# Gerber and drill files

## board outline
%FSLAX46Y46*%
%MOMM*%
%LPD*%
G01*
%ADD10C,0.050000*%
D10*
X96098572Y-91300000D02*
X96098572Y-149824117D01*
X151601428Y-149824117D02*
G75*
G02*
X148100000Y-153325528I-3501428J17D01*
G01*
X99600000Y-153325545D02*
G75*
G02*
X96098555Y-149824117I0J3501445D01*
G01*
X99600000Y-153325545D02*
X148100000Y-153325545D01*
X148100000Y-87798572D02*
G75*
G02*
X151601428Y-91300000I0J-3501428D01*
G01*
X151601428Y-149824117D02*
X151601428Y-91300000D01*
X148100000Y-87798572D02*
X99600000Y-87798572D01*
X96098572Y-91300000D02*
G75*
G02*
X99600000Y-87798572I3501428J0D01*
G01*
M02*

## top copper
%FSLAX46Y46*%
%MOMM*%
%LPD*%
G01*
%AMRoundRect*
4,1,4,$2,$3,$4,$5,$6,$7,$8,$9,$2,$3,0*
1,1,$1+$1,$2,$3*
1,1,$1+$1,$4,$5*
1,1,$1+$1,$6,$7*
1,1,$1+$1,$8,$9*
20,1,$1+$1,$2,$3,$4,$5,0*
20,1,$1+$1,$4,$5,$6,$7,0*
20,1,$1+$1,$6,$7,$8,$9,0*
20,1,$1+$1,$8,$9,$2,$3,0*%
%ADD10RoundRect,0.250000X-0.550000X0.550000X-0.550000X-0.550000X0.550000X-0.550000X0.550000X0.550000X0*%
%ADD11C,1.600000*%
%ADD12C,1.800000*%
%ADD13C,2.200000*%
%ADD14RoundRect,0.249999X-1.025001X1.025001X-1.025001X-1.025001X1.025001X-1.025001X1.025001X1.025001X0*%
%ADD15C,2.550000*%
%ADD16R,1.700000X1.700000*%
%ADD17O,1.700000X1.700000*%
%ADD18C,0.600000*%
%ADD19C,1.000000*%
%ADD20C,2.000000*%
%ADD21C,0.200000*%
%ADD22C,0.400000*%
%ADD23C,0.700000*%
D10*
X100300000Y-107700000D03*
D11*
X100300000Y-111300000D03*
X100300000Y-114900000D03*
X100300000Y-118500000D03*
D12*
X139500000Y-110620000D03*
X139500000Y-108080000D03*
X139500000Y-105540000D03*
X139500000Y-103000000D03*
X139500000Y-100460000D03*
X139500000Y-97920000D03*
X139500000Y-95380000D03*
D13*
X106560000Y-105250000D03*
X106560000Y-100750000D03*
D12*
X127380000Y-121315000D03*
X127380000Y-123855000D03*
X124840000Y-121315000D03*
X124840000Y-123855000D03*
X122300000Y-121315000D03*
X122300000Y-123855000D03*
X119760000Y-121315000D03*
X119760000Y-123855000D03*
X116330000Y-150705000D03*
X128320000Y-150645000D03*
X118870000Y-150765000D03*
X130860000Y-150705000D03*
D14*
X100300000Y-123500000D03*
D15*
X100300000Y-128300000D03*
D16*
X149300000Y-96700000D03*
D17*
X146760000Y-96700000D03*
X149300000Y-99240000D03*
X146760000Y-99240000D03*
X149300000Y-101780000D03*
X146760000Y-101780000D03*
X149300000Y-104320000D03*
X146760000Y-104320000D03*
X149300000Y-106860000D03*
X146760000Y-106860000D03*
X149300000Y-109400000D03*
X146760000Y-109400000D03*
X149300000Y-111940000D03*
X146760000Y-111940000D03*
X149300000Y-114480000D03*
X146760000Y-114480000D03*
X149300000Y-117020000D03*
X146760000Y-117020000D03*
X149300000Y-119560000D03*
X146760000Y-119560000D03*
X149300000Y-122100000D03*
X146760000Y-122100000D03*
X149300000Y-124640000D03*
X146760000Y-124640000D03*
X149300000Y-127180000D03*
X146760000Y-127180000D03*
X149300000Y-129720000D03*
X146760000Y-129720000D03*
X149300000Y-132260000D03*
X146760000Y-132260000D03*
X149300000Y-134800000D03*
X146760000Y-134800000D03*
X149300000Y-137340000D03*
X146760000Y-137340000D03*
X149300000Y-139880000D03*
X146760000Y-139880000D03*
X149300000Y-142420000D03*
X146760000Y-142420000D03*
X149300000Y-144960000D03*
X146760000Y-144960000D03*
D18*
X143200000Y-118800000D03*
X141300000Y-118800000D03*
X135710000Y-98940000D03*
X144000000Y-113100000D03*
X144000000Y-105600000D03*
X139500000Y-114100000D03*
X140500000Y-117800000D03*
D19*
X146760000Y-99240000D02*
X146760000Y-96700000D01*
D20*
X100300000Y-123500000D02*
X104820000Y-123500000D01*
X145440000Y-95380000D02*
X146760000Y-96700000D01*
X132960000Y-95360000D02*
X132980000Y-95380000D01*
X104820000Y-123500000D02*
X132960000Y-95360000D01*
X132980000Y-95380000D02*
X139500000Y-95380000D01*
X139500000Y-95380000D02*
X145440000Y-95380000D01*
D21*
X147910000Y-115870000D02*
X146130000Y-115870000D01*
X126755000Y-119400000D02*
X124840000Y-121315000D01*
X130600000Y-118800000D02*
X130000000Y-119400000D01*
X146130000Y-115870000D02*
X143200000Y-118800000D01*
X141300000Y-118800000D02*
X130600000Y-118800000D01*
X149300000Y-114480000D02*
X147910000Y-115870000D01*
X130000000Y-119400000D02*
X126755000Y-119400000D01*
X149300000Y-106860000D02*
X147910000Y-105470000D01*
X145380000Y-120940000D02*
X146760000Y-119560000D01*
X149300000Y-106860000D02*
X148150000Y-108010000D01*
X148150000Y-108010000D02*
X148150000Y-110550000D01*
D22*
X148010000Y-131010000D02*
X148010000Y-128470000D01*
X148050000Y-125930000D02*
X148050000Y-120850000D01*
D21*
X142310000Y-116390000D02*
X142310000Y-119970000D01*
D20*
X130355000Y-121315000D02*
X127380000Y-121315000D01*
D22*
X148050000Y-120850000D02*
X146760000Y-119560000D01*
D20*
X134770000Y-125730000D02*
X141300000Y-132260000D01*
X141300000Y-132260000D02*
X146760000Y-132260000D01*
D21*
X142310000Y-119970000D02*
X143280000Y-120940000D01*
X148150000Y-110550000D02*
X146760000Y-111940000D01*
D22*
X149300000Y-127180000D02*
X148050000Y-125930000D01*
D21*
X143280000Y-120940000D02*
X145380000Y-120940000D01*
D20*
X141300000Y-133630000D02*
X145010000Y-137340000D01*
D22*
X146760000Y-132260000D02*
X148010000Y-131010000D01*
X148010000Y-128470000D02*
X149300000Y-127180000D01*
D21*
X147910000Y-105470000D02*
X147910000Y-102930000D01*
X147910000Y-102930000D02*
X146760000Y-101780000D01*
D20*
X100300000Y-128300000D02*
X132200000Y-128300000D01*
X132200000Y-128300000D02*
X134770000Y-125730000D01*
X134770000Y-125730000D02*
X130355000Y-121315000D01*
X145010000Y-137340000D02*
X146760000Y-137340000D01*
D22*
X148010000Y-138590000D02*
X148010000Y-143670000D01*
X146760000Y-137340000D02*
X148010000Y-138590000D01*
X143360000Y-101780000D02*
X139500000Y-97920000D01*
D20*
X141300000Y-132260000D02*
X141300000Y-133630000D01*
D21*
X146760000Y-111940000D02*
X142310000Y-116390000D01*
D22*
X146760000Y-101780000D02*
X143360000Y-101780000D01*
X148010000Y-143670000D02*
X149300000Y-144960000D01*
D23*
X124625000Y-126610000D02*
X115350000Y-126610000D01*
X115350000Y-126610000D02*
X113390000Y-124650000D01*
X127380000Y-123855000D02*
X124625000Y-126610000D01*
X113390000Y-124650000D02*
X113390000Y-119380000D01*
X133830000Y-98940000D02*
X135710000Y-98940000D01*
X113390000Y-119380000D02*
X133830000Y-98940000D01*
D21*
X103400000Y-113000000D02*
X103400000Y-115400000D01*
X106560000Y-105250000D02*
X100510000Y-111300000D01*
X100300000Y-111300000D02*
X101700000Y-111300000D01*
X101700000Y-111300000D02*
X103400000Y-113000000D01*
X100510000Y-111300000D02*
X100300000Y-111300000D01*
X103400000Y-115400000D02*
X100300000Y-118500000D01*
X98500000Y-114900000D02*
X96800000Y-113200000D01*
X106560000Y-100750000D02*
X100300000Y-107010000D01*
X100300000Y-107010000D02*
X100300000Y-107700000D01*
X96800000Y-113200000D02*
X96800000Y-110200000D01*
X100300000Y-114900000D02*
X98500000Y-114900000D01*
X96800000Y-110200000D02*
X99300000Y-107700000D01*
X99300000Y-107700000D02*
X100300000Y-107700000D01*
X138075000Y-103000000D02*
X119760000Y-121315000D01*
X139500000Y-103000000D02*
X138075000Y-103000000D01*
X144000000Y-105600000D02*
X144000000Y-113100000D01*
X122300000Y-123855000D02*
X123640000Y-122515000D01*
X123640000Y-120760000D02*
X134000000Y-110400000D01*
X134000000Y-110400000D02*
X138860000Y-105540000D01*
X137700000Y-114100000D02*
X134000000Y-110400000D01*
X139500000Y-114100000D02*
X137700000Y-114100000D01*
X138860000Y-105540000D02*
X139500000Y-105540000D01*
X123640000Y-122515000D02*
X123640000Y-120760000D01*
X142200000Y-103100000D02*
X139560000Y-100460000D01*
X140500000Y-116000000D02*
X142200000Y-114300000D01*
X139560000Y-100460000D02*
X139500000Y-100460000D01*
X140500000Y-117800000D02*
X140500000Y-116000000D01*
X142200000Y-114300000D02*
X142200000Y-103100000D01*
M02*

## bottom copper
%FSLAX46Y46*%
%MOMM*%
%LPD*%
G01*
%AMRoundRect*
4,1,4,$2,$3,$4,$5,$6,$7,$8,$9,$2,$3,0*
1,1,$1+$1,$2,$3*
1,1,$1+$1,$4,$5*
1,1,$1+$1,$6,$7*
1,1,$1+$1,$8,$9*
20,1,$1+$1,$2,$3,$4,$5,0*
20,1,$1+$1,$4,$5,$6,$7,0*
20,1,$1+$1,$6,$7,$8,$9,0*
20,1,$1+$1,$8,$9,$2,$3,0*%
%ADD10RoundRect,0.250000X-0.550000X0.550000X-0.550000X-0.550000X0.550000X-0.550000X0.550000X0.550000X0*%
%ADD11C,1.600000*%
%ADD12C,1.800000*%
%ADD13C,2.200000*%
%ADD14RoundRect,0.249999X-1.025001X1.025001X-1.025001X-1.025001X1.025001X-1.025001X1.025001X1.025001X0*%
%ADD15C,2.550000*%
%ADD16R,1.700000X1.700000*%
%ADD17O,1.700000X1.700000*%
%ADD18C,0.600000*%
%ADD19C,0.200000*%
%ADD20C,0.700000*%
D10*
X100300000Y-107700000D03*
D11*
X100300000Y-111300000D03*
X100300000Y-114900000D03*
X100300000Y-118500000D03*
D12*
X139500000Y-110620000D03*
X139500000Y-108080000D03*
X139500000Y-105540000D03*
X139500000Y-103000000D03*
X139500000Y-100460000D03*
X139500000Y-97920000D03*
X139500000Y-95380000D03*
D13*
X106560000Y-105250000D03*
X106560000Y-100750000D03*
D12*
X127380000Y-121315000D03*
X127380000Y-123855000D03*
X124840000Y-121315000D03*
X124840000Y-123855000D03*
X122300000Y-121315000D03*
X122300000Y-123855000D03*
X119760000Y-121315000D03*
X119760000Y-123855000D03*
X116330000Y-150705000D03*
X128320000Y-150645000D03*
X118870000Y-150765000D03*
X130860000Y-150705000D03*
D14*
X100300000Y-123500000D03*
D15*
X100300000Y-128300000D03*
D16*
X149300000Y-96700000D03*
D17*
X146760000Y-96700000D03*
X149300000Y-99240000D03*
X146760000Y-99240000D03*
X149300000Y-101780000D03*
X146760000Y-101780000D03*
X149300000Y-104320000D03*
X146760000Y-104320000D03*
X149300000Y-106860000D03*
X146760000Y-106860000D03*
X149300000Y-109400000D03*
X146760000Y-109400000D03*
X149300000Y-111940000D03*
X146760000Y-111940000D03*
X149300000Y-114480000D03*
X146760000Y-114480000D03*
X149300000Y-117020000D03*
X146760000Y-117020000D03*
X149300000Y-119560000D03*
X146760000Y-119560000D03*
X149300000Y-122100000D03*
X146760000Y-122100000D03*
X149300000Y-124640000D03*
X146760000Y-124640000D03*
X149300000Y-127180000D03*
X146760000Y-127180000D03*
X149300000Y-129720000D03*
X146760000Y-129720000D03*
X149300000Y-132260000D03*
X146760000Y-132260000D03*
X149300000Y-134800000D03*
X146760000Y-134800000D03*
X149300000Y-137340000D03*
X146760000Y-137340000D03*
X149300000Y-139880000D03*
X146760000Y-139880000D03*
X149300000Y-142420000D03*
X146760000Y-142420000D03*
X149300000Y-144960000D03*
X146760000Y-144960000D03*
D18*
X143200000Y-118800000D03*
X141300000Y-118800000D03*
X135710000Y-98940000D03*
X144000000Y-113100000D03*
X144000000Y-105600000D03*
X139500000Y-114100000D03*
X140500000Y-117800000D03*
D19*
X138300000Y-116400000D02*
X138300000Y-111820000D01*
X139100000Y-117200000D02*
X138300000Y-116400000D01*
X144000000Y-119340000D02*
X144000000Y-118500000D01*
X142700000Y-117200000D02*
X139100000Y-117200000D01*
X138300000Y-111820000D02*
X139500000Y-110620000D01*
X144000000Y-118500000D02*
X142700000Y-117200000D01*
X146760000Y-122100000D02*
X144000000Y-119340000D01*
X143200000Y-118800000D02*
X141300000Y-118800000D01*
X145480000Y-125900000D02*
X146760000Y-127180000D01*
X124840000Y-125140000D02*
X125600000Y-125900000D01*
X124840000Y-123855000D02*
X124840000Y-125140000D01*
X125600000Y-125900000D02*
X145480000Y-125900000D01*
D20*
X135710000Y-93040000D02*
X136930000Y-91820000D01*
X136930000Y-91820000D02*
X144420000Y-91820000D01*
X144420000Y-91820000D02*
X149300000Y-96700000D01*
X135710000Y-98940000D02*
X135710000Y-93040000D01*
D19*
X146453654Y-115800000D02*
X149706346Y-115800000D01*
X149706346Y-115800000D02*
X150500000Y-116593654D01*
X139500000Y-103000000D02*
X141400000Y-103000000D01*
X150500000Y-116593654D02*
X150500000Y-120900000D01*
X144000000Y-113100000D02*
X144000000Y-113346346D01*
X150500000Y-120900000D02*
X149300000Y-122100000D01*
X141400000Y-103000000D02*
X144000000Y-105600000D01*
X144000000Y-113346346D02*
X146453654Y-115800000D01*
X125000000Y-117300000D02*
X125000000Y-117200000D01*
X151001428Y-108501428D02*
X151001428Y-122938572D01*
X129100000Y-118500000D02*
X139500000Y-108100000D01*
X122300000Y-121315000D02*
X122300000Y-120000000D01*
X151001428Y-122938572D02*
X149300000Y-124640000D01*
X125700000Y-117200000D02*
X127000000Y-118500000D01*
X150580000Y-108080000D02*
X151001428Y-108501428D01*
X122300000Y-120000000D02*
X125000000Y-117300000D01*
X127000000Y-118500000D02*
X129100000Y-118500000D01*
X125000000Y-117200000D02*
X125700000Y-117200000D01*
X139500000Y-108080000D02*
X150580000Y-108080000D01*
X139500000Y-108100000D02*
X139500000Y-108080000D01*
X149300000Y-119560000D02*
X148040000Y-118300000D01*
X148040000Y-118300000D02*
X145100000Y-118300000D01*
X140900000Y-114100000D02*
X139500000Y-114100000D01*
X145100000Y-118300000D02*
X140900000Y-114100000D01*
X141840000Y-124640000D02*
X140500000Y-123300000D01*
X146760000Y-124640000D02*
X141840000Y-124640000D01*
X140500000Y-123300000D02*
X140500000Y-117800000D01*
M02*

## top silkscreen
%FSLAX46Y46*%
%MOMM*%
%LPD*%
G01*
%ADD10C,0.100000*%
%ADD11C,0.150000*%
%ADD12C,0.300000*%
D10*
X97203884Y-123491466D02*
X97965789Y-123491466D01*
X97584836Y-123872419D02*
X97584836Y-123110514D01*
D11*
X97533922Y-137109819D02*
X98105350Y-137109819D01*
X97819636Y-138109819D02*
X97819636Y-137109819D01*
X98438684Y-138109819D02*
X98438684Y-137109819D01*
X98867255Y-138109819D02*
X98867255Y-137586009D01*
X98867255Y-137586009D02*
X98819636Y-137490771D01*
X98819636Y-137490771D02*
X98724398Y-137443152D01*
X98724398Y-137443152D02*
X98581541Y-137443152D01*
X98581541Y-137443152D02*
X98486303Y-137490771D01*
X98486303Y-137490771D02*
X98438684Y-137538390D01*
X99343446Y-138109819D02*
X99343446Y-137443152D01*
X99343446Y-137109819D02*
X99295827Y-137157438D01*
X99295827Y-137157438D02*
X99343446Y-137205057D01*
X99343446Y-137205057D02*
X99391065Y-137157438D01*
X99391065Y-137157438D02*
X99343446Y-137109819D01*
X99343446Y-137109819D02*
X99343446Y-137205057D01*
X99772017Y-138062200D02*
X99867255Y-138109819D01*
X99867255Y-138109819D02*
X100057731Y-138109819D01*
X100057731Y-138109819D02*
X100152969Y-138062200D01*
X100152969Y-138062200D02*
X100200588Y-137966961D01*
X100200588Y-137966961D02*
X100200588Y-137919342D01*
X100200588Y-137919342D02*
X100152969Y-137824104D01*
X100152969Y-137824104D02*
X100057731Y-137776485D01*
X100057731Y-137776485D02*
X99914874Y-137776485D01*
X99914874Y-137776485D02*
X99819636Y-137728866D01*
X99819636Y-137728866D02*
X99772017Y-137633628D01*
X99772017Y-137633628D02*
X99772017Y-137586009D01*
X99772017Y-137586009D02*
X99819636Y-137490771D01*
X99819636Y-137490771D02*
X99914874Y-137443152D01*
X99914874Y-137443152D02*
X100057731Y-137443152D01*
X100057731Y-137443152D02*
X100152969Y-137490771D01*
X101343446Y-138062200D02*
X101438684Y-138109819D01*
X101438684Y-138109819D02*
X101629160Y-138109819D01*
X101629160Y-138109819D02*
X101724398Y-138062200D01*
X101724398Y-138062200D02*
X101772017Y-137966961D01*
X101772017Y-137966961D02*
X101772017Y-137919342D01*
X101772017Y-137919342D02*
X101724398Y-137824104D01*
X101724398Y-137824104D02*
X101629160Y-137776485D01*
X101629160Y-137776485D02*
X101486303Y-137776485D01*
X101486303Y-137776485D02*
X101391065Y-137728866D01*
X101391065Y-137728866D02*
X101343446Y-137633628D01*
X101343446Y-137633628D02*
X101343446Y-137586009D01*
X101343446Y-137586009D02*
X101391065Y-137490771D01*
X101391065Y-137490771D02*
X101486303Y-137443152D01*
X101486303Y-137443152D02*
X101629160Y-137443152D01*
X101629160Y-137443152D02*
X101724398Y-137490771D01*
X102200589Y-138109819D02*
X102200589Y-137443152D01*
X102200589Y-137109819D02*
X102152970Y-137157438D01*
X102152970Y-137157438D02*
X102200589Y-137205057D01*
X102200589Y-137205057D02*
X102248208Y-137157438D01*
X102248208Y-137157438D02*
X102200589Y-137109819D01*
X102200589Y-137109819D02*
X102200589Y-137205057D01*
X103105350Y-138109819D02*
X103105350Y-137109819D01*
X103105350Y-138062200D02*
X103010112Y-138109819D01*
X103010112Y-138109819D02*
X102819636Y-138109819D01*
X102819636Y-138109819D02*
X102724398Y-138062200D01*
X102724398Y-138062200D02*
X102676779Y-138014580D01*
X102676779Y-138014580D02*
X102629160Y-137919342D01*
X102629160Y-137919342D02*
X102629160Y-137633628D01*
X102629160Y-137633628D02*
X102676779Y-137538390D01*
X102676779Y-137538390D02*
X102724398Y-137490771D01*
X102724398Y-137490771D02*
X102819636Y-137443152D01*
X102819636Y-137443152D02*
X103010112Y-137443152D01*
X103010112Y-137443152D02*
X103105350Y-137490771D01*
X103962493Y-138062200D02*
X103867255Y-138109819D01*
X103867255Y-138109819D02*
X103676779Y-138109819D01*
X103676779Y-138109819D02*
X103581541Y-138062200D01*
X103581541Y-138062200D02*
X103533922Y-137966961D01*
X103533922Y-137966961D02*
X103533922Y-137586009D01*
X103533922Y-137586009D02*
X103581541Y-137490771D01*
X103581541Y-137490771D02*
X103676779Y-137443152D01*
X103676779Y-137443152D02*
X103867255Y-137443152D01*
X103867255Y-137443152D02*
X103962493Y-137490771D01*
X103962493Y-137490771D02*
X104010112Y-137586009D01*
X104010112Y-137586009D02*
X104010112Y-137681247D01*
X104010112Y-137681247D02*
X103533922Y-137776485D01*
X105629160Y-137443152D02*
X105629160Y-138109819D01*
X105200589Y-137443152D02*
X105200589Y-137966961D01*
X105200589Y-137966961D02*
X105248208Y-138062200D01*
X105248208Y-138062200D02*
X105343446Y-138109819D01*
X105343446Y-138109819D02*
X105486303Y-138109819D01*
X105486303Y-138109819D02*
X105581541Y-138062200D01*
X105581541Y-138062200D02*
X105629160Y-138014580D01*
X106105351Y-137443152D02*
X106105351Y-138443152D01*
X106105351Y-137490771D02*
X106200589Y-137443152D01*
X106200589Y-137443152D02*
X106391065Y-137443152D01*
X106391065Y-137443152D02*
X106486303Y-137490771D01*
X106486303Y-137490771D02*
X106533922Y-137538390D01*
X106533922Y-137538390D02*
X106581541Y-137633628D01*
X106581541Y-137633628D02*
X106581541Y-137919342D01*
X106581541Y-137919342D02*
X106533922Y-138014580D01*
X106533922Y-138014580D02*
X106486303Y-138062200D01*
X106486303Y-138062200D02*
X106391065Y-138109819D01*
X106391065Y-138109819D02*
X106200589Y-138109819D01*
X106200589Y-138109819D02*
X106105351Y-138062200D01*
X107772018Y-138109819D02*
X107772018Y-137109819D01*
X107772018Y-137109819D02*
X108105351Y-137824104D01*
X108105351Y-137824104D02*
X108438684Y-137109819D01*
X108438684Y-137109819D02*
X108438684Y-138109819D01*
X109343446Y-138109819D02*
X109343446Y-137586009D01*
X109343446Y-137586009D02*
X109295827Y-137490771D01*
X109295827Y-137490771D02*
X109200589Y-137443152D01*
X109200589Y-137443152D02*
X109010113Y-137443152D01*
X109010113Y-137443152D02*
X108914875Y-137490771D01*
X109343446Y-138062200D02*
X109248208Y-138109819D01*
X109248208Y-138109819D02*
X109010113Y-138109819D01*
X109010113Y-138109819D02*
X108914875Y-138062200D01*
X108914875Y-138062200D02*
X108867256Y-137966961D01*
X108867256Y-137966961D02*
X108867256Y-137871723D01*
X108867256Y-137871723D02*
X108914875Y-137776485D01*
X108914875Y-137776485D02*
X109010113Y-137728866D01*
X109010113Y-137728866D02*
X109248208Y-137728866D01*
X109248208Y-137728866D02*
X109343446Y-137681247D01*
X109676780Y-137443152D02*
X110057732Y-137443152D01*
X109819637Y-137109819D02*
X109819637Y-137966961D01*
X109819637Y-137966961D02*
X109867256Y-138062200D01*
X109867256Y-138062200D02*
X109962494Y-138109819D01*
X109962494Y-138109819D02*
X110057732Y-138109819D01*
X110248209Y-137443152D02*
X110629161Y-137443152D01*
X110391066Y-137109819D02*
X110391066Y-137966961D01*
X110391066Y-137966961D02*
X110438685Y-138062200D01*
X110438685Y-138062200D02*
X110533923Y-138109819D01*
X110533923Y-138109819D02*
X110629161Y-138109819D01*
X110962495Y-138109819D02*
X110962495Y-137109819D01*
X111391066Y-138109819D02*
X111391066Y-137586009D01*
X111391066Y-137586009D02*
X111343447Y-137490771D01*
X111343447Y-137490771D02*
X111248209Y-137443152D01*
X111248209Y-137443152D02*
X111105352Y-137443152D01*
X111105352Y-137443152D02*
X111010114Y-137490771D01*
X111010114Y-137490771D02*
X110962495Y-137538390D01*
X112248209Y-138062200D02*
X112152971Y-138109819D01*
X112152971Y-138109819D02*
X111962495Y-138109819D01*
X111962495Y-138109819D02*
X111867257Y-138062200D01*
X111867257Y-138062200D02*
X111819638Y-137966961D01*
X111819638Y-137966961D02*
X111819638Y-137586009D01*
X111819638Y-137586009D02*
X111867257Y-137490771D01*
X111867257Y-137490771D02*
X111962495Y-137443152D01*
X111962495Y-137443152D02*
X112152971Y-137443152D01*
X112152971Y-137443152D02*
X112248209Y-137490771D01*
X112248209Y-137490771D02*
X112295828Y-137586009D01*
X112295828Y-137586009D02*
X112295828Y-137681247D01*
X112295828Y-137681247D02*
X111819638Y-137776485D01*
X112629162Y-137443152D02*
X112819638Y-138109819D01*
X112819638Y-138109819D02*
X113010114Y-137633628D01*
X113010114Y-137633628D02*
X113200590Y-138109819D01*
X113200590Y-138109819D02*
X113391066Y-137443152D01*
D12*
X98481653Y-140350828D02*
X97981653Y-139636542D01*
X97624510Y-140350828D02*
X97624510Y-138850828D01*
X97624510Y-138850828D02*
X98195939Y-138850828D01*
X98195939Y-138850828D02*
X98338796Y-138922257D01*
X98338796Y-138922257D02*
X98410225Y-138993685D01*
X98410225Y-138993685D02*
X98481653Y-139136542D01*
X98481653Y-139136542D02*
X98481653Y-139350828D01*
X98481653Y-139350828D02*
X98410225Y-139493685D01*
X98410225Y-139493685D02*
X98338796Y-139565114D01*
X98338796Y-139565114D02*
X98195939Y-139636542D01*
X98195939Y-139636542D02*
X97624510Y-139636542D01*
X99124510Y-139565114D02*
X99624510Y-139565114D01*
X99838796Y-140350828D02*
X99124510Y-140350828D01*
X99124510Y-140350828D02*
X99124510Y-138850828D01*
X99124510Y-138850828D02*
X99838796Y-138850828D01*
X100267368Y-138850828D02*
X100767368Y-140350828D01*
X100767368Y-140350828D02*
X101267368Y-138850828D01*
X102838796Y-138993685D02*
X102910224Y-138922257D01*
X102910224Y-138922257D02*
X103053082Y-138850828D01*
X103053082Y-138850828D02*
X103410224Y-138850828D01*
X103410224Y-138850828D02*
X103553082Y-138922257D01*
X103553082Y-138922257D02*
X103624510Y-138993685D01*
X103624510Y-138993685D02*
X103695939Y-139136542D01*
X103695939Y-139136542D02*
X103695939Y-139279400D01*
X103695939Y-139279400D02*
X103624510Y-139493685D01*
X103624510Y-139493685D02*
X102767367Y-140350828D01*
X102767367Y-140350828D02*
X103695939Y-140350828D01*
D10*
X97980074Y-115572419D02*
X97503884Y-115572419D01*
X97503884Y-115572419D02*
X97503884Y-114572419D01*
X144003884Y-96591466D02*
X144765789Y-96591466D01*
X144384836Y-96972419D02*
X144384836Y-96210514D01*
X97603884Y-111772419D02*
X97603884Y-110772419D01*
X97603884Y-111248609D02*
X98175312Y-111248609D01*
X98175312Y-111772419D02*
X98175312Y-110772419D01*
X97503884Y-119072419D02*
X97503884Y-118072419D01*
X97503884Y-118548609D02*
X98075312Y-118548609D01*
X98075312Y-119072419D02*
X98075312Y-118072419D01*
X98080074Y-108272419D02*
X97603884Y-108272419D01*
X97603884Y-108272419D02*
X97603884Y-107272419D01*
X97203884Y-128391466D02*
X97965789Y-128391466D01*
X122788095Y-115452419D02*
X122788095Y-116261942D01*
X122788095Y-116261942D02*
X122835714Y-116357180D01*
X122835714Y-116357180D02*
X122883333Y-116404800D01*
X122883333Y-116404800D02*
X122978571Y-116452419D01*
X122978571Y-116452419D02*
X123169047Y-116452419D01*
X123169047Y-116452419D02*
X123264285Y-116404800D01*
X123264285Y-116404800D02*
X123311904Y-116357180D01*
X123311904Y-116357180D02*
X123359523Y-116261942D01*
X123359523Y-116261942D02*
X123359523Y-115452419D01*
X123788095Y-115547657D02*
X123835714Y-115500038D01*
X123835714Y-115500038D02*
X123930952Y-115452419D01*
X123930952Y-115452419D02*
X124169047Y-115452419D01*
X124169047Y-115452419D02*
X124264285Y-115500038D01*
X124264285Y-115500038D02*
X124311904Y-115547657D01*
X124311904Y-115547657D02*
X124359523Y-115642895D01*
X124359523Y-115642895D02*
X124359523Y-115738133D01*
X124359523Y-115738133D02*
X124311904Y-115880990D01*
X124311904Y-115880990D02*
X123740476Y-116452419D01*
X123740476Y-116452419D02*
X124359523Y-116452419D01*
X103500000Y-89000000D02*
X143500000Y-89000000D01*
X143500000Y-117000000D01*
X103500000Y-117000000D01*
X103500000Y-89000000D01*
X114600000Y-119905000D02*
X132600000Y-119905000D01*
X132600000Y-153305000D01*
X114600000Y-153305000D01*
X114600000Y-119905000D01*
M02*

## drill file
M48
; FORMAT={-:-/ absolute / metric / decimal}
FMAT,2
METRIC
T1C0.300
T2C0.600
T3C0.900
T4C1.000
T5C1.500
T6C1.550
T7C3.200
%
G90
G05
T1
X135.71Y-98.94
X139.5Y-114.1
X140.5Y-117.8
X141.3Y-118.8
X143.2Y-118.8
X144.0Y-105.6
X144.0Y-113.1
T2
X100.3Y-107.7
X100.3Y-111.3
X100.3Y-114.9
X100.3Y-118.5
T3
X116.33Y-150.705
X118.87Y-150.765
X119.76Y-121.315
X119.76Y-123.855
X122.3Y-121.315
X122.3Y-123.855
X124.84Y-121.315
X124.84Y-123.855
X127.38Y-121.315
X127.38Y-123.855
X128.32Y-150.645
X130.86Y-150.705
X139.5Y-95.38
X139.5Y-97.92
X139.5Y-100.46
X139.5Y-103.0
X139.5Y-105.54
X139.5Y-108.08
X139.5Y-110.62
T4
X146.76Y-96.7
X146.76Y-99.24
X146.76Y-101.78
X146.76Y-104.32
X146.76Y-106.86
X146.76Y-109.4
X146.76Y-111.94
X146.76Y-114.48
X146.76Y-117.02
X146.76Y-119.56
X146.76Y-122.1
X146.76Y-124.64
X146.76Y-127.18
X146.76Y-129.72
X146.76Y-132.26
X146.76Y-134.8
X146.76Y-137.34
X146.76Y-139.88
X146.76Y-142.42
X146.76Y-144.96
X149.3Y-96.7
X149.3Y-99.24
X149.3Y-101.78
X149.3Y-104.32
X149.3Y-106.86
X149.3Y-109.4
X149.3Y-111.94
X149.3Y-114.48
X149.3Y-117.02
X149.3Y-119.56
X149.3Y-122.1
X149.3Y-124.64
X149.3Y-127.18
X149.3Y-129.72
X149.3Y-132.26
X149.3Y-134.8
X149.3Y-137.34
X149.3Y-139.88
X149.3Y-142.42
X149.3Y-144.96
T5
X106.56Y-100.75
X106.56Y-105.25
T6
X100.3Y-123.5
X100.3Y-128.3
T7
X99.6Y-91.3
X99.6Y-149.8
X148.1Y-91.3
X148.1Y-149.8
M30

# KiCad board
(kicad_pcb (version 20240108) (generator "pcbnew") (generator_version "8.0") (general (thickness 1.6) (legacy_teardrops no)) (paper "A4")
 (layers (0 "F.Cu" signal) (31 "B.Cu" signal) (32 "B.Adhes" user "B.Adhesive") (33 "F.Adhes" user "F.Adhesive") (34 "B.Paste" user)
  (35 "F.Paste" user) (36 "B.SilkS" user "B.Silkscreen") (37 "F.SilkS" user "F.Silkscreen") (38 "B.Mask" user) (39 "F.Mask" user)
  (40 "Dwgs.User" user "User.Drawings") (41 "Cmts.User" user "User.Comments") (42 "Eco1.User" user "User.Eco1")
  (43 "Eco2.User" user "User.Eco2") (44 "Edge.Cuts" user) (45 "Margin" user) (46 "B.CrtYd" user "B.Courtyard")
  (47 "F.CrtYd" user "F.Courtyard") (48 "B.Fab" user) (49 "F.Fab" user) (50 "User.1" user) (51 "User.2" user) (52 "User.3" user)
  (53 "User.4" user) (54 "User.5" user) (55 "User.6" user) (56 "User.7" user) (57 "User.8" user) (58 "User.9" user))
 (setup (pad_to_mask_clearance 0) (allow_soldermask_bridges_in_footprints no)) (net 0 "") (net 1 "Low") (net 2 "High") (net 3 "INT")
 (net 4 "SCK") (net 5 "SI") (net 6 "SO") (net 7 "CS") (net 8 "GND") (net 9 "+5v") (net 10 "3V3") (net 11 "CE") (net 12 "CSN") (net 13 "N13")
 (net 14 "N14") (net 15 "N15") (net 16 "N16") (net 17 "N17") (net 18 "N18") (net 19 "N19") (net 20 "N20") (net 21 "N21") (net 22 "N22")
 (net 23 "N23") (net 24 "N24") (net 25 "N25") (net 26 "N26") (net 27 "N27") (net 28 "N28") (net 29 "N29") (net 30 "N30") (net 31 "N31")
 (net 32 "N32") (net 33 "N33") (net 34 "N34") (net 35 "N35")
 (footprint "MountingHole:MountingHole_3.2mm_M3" (layer "F.Cu") (at 148.1 91.3 180)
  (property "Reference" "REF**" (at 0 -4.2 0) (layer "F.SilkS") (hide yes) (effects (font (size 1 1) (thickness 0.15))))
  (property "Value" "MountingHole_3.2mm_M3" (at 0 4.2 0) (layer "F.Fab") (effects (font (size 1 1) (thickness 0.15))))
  (pad "" np_thru_hole circle (at 0 0 180) (size 3.2 3.2) (drill 3.2) (layers "*.Cu" "*.Mask")))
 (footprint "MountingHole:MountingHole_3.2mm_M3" (layer "F.Cu") (at 99.6 91.3 180)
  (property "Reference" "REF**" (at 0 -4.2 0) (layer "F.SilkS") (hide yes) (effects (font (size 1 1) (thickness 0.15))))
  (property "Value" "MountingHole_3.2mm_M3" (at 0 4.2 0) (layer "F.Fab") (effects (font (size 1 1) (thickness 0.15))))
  (pad "" np_thru_hole circle (at 0 0 180) (size 3.2 3.2) (drill 3.2) (layers "*.Cu" "*.Mask")))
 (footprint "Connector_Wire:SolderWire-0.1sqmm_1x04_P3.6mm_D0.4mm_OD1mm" (layer "F.Cu") (at 100.3 107.7 -90)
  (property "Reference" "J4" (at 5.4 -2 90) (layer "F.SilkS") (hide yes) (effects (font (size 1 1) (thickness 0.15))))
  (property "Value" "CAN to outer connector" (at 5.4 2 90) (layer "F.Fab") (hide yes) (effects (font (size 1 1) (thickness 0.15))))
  (pad "1" thru_hole roundrect (at 0 0 270) (size 1.6 1.6) (drill 0.6) (layers "*.Cu" "*.Mask") (remove_unused_layers no)
   (roundrect_rratio 0.15625) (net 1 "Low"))
  (pad "2" thru_hole circle (at 3.6 0 270) (size 1.6 1.6) (drill 0.6) (layers "*.Cu" "*.Mask") (remove_unused_layers no) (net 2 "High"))
  (pad "3" thru_hole circle (at 7.2 0 270) (size 1.6 1.6) (drill 0.6) (layers "*.Cu" "*.Mask") (remove_unused_layers no) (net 1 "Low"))
  (pad "4" thru_hole circle (at 10.8 0 270) (size 1.6 1.6) (drill 0.6) (layers "*.Cu" "*.Mask") (remove_unused_layers no) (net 2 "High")))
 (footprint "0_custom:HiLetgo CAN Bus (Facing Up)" (layer "F.Cu") (at 129.55 100.6 180)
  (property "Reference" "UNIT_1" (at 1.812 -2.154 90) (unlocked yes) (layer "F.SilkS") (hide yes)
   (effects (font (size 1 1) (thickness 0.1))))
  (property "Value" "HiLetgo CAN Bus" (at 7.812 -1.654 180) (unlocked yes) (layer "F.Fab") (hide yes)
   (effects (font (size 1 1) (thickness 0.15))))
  (fp_rect (start -13.95 -16.4) (end 26.05 11.6) (stroke (width 0.1) (type default)) (fill none) (layer "F.SilkS"))
  (pad "1" thru_hole circle (at -9.95 -10.02) (size 1.8 1.8) (drill 0.9) (layers "*.Cu" "*.Mask") (remove_unused_layers no) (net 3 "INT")
   (solder_mask_margin 0.102))
  (pad "2" thru_hole circle (at -9.95 -7.48) (size 1.8 1.8) (drill 0.9) (layers "*.Cu" "*.Mask") (remove_unused_layers no) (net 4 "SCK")
   (solder_mask_margin 0.102))
  (pad "3" thru_hole circle (at -9.95 -4.94) (size 1.8 1.8) (drill 0.9) (layers "*.Cu" "*.Mask") (remove_unused_layers no) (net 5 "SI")
   (solder_mask_margin 0.102))
  (pad "4" thru_hole circle (at -9.95 -2.4) (size 1.8 1.8) (drill 0.9) (layers "*.Cu" "*.Mask") (remove_unused_layers no) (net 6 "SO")
   (solder_mask_margin 0.102))
  (pad "5" thru_hole circle (at -9.95 0.14) (size 1.8 1.8) (drill 0.9) (layers "*.Cu" "*.Mask") (remove_unused_layers no) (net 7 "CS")
   (solder_mask_margin 0.102))
  (pad "6" thru_hole circle (at -9.95 2.68) (size 1.8 1.8) (drill 0.9) (layers "*.Cu" "*.Mask") (remove_unused_layers no) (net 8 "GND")
   (solder_mask_margin 0.102))
  (pad "7" thru_hole circle (at -9.95 5.22) (size 1.8 1.8) (drill 0.9) (layers "*.Cu" "*.Mask") (remove_unused_layers no) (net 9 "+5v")
   (solder_mask_margin 0.102))
  (pad "8" thru_hole circle (at 22.99 -4.65) (size 2.2 2.2) (drill 1.5) (layers "*.Cu" "*.Mask") (remove_unused_layers no) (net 2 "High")
   (solder_mask_margin 0.102))
  (pad "9" thru_hole circle (at 22.99 -0.15) (size 2.2 2.2) (drill 1.5) (layers "*.Cu" "*.Mask") (remove_unused_layers no) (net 1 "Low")
   (solder_mask_margin 0.102)))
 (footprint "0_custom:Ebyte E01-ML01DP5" (layer "F.Cu") (at 123.55 116.495)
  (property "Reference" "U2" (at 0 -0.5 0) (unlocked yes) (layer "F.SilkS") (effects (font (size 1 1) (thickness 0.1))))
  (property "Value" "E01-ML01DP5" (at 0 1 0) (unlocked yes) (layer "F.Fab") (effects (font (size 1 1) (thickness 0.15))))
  (fp_rect (start -8.95 3.41) (end 9.05 36.81) (stroke (width 0.1) (type default)) (fill none) (layer "F.SilkS"))
  (pad "1" thru_hole circle (at 3.83 4.82 180) (size 1.8 1.8) (drill 0.9) (layers "*.Cu" "*.Mask") (remove_unused_layers no) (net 8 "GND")
   (solder_mask_margin 0.102))
  (pad "2" thru_hole circle (at 3.83 7.36 180) (size 1.8 1.8) (drill 0.9) (layers "*.Cu" "*.Mask") (remove_unused_layers no) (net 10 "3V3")
   (solder_mask_margin 0.102))
  (pad "3" thru_hole circle (at 1.29 4.82 180) (size 1.8 1.8) (drill 0.9) (layers "*.Cu" "*.Mask") (remove_unused_layers no) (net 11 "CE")
   (solder_mask_margin 0.102))
  (pad "4" thru_hole circle (at 1.29 7.36 180) (size 1.8 1.8) (drill 0.9) (layers "*.Cu" "*.Mask") (remove_unused_layers no) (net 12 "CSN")
   (solder_mask_margin 0.102))
  (pad "5" thru_hole circle (at -1.25 4.82 180) (size 1.8 1.8) (drill 0.9) (layers "*.Cu" "*.Mask") (remove_unused_layers no) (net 4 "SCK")
   (solder_mask_margin 0.102))
  (pad "6" thru_hole circle (at -1.25 7.36 180) (size 1.8 1.8) (drill 0.9) (layers "*.Cu" "*.Mask") (remove_unused_layers no) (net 5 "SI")
   (solder_mask_margin 0.102))
  (pad "7" thru_hole circle (at -3.79 4.82 90) (size 1.8 1.8) (drill 0.9) (layers "*.Cu" "*.Mask") (remove_unused_layers no) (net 6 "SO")
   (solder_mask_margin 0.102))
  (pad "8" thru_hole circle (at -3.79 7.36 90) (size 1.8 1.8) (drill 0.9) (layers "*.Cu" "*.Mask") (remove_unused_layers no) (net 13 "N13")
   (solder_mask_margin 0.102))
  (pad "9" thru_hole circle (at -7.22 34.21 270) (size 1.8 1.8) (drill 0.9) (layers "*.Cu" "*.Mask") (remove_unused_layers no)
   (solder_mask_margin 0.102))
  (pad "9" thru_hole circle (at 4.77 34.15 270) (size 1.8 1.8) (drill 0.9) (layers "*.Cu" "*.Mask") (remove_unused_layers no)
   (solder_mask_margin 0.102))
  (pad "10" thru_hole circle (at -4.68 34.27 270) (size 1.8 1.8) (drill 0.9) (layers "*.Cu" "*.Mask") (remove_unused_layers no)
   (solder_mask_margin 0.102))
  (pad "10" thru_hole circle (at 7.31 34.21 270) (size 1.8 1.8) (drill 0.9) (layers "*.Cu" "*.Mask") (remove_unused_layers no)
   (solder_mask_margin 0.102)))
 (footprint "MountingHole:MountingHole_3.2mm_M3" (layer "F.Cu") (at 99.6 149.8)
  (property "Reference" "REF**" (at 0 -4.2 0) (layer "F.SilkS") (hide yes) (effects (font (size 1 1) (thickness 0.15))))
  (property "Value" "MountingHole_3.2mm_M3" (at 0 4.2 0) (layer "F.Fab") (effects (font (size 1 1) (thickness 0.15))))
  (pad "" np_thru_hole circle (at 0 0) (size 3.2 3.2) (drill 3.2) (layers "*.Cu" "*.Mask")))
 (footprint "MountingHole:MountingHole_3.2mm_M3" (layer "F.Cu") (at 148.1 149.8)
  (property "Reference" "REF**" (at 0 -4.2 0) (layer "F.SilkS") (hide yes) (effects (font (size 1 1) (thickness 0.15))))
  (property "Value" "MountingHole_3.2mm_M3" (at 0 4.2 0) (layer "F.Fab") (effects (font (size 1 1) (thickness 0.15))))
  (pad "" np_thru_hole circle (at 0 0) (size 3.2 3.2) (drill 3.2) (layers "*.Cu" "*.Mask")))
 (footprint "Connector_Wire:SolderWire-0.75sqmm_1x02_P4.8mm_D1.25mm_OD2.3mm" (layer "F.Cu") (at 100.3 123.5 -90)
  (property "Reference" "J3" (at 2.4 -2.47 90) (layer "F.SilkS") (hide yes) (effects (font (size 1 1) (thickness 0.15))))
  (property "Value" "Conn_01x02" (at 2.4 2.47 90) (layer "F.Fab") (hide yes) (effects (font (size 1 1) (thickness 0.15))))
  (pad "1" thru_hole roundrect (at 0 0 270) (size 2.55 2.55) (drill 1.55) (layers "*.Cu" "*.Mask") (remove_unused_layers no)
   (roundrect_rratio 0.098039) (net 9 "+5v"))
  (pad "2" thru_hole circle (at 4.8 0 270) (size 2.55 2.55) (drill 1.55) (layers "*.Cu" "*.Mask") (remove_unused_layers no) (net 8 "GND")))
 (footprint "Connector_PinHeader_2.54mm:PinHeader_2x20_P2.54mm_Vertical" (layer "B.Cu") (at 149.3 96.7 180)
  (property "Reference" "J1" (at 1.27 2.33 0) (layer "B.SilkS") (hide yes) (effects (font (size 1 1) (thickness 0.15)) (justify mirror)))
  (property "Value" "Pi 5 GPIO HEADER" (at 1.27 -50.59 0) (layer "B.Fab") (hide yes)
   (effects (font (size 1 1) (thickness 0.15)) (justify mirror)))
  (pad "1" thru_hole rect (at 0 0 180) (size 1.7 1.7) (drill 1) (layers "*.Cu" "*.Mask") (remove_unused_layers no) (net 10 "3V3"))
  (pad "2" thru_hole oval (at 2.54 0 180) (size 1.7 1.7) (drill 1) (layers "*.Cu" "*.Mask") (remove_unused_layers no) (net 9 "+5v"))
  (pad "3" thru_hole oval (at 0 -2.54 180) (size 1.7 1.7) (drill 1) (layers "*.Cu" "*.Mask") (remove_unused_layers no) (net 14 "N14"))
  (pad "4" thru_hole oval (at 2.54 -2.54 180) (size 1.7 1.7) (drill 1) (layers "*.Cu" "*.Mask") (remove_unused_layers no) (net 9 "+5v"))
  (pad "5" thru_hole oval (at 0 -5.08 180) (size 1.7 1.7) (drill 1) (layers "*.Cu" "*.Mask") (remove_unused_layers no) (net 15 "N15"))
  (pad "6" thru_hole oval (at 2.54 -5.08 180) (size 1.7 1.7) (drill 1) (layers "*.Cu" "*.Mask") (remove_unused_layers no) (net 8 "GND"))
  (pad "7" thru_hole oval (at 0 -7.62 180) (size 1.7 1.7) (drill 1) (layers "*.Cu" "*.Mask") (remove_unused_layers no) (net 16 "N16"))
  (pad "8" thru_hole oval (at 2.54 -7.62 180) (size 1.7 1.7) (drill 1) (layers "*.Cu" "*.Mask") (remove_unused_layers no) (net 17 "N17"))
  (pad "9" thru_hole oval (at 0 -10.16 180) (size 1.7 1.7) (drill 1) (layers "*.Cu" "*.Mask") (remove_unused_layers no) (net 8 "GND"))
  (pad "10" thru_hole oval (at 2.54 -10.16 180) (size 1.7 1.7) (drill 1) (layers "*.Cu" "*.Mask") (remove_unused_layers no) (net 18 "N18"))
  (pad "11" thru_hole oval (at 0 -12.7 180) (size 1.7 1.7) (drill 1) (layers "*.Cu" "*.Mask") (remove_unused_layers no) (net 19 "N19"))
  (pad "12" thru_hole oval (at 2.54 -12.7 180) (size 1.7 1.7) (drill 1) (layers "*.Cu" "*.Mask") (remove_unused_layers no) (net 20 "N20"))
  (pad "13" thru_hole oval (at 0 -15.24 180) (size 1.7 1.7) (drill 1) (layers "*.Cu" "*.Mask") (remove_unused_layers no) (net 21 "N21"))
  (pad "14" thru_hole oval (at 2.54 -15.24 180) (size 1.7 1.7) (drill 1) (layers "*.Cu" "*.Mask") (remove_unused_layers no) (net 8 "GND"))
  (pad "15" thru_hole oval (at 0 -17.78 180) (size 1.7 1.7) (drill 1) (layers "*.Cu" "*.Mask") (remove_unused_layers no) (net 11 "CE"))
  (pad "16" thru_hole oval (at 2.54 -17.78 180) (size 1.7 1.7) (drill 1) (layers "*.Cu" "*.Mask") (remove_unused_layers no) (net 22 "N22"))
  (pad "17" thru_hole oval (at 0 -20.32 180) (size 1.7 1.7) (drill 1) (layers "*.Cu" "*.Mask") (remove_unused_layers no) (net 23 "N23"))
  (pad "18" thru_hole oval (at 2.54 -20.32 180) (size 1.7 1.7) (drill 1) (layers "*.Cu" "*.Mask") (remove_unused_layers no) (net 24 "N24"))
  (pad "19" thru_hole oval (at 0 -22.86 180) (size 1.7 1.7) (drill 1) (layers "*.Cu" "*.Mask") (remove_unused_layers no) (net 5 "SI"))
  (pad "20" thru_hole oval (at 2.54 -22.86 180) (size 1.7 1.7) (drill 1) (layers "*.Cu" "*.Mask") (remove_unused_layers no) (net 8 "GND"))
  (pad "21" thru_hole oval (at 0 -25.4 180) (size 1.7 1.7) (drill 1) (layers "*.Cu" "*.Mask") (remove_unused_layers no) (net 6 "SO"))
  (pad "22" thru_hole oval (at 2.54 -25.4 180) (size 1.7 1.7) (drill 1) (layers "*.Cu" "*.Mask") (remove_unused_layers no) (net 3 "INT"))
  (pad "23" thru_hole oval (at 0 -27.94 180) (size 1.7 1.7) (drill 1) (layers "*.Cu" "*.Mask") (remove_unused_layers no) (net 4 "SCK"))
  (pad "24" thru_hole oval (at 2.54 -27.94 180) (size 1.7 1.7) (drill 1) (layers "*.Cu" "*.Mask") (remove_unused_layers no) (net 7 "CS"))
  (pad "25" thru_hole oval (at 0 -30.48 180) (size 1.7 1.7) (drill 1) (layers "*.Cu" "*.Mask") (remove_unused_layers no) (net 8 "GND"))
  (pad "26" thru_hole oval (at 2.54 -30.48 180) (size 1.7 1.7) (drill 1) (layers "*.Cu" "*.Mask") (remove_unused_layers no) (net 12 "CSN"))
  (pad "27" thru_hole oval (at 0 -33.02 180) (size 1.7 1.7) (drill 1) (layers "*.Cu" "*.Mask") (remove_unused_layers no) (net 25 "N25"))
  (pad "28" thru_hole oval (at 2.54 -33.02 180) (size 1.7 1.7) (drill 1) (layers "*.Cu" "*.Mask") (remove_unused_layers no) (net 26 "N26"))
  (pad "29" thru_hole oval (at 0 -35.56 180) (size 1.7 1.7) (drill 1) (layers "*.Cu" "*.Mask") (remove_unused_layers no) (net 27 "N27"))
  (pad "30" thru_hole oval (at 2.54 -35.56 180) (size 1.7 1.7) (drill 1) (layers "*.Cu" "*.Mask") (remove_unused_layers no) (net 8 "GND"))
  (pad "31" thru_hole oval (at 0 -38.1 180) (size 1.7 1.7) (drill 1) (layers "*.Cu" "*.Mask") (remove_unused_layers no) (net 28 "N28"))
  (pad "32" thru_hole oval (at 2.54 -38.1 180) (size 1.7 1.7) (drill 1) (layers "*.Cu" "*.Mask") (remove_unused_layers no) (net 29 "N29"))
  (pad "33" thru_hole oval (at 0 -40.64 180) (size 1.7 1.7) (drill 1) (layers "*.Cu" "*.Mask") (remove_unused_layers no) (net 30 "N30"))
  (pad "34" thru_hole oval (at 2.54 -40.64 180) (size 1.7 1.7) (drill 1) (layers "*.Cu" "*.Mask") (remove_unused_layers no) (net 8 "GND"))
  (pad "35" thru_hole oval (at 0 -43.18 180) (size 1.7 1.7) (drill 1) (layers "*.Cu" "*.Mask") (remove_unused_layers no) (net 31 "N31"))
  (pad "36" thru_hole oval (at 2.54 -43.18 180) (size 1.7 1.7) (drill 1) (layers "*.Cu" "*.Mask") (remove_unused_layers no) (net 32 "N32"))
  (pad "37" thru_hole oval (at 0 -45.72 180) (size 1.7 1.7) (drill 1) (layers "*.Cu" "*.Mask") (remove_unused_layers no) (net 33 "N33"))
  (pad "38" thru_hole oval (at 2.54 -45.72 180) (size 1.7 1.7) (drill 1) (layers "*.Cu" "*.Mask") (remove_unused_layers no) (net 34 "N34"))
  (pad "39" thru_hole oval (at 0 -48.26 180) (size 1.7 1.7) (drill 1) (layers "*.Cu" "*.Mask") (remove_unused_layers no) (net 8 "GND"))
  (pad "40" thru_hole oval (at 2.54 -48.26 180) (size 1.7 1.7) (drill 1) (layers "*.Cu" "*.Mask") (remove_unused_layers no) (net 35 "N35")))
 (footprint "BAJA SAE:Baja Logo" (layer "B.Cu") (at 122.9 102.7 180)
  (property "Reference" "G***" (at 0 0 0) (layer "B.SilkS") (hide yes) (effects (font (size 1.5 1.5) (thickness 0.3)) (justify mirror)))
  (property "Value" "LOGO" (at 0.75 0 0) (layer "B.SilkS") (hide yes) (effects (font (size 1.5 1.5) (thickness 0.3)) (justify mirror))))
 (gr_line (start 96.098572 91.3) (end 96.098572 149.824117) (stroke (width 0.05) (type default)) (layer "Edge.Cuts"))
 (gr_arc (start 151.601428 149.824117) (mid 150.575883 152.3) (end 148.1 153.325545) (locked yes) (stroke (width 0.05) (type default))
  (layer "Edge.Cuts"))
 (gr_arc (start 99.6 153.325545) (mid 97.124117 152.3) (end 96.098572 149.824117) (stroke (width 0.05) (type default)) (layer "Edge.Cuts"))
 (gr_line (start 99.6 153.325545) (end 148.1 153.325545) (stroke (width 0.05) (type default)) (layer "Edge.Cuts"))
 (gr_arc (start 148.1 87.798572) (mid 150.575883 88.824117) (end 151.601428 91.3) (locked yes) (stroke (width 0.05) (type default))
  (layer "Edge.Cuts"))
 (gr_line (start 151.601428 149.824117) (end 151.601428 91.3) (stroke (width 0.05) (type default)) (layer "Edge.Cuts"))
 (gr_line (start 148.1 87.798572) (end 99.6 87.798572) (stroke (width 0.05) (type default)) (layer "Edge.Cuts"))
 (gr_arc (start 96.098572 91.3) (mid 97.124117 88.824117) (end 99.6 87.798572) (locked yes) (stroke (width 0.05) (type default))
  (layer "Edge.Cuts"))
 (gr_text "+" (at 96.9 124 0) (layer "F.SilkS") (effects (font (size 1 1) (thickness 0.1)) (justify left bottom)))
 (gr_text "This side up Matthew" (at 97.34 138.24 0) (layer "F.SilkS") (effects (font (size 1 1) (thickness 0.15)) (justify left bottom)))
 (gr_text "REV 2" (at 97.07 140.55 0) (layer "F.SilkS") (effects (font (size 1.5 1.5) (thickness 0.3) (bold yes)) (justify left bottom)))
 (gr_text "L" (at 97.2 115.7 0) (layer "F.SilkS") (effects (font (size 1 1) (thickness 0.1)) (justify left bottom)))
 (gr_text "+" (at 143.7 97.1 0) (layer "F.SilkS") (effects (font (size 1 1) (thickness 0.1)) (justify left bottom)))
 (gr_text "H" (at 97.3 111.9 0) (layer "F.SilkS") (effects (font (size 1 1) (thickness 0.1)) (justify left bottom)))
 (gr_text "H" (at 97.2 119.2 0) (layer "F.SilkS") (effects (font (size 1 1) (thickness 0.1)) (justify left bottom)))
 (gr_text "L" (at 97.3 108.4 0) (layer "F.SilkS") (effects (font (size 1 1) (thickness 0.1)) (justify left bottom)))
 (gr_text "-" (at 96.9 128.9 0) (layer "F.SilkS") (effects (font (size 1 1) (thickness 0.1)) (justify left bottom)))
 (segment (start 138.3 116.4) (end 138.3 111.82) (width 0.2) (layer "B.Cu") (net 3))
 (segment (start 139.1 117.2) (end 138.3 116.4) (width 0.2) (layer "B.Cu") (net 3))
 (segment (start 144 119.34) (end 144 118.5) (width 0.2) (layer "B.Cu") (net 3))
 (segment (start 142.7 117.2) (end 139.1 117.2) (width 0.2) (layer "B.Cu") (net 3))
 (segment (start 138.3 111.82) (end 139.5 110.62) (width 0.2) (layer "B.Cu") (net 3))
 (segment (start 144 118.5) (end 142.7 117.2) (width 0.2) (layer "B.Cu") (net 3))
 (segment (start 146.76 122.1) (end 144 119.34) (width 0.2) (layer "B.Cu") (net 3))
 (segment (start 146.76 99.24) (end 146.76 96.7) (width 1) (layer "F.Cu") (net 9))
 (segment (start 100.3 123.5) (end 104.82 123.5) (width 2) (layer "F.Cu") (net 9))
 (segment (start 145.44 95.38) (end 146.76 96.7) (width 2) (layer "F.Cu") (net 9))
 (segment (start 132.96 95.36) (end 132.98 95.38) (width 2) (layer "F.Cu") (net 9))
 (segment (start 104.82 123.5) (end 132.96 95.36) (width 2) (layer "F.Cu") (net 9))
 (segment (start 132.98 95.38) (end 139.5 95.38) (width 2) (layer "F.Cu") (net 9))
 (segment (start 139.5 95.38) (end 145.44 95.38) (width 2) (layer "F.Cu") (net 9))
 (segment (start 147.91 115.87) (end 146.13 115.87) (width 0.2) (layer "F.Cu") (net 11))
 (segment (start 126.755 119.4) (end 124.84 121.315) (width 0.2) (layer "F.Cu") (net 11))
 (segment (start 130.6 118.8) (end 130 119.4) (width 0.2) (layer "F.Cu") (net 11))
 (segment (start 146.13 115.87) (end 143.2 118.8) (width 0.2) (layer "F.Cu") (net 11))
 (segment (start 141.3 118.8) (end 130.6 118.8) (width 0.2) (layer "F.Cu") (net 11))
 (segment (start 149.3 114.48) (end 147.91 115.87) (width 0.2) (layer "F.Cu") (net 11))
 (segment (start 130 119.4) (end 126.755 119.4) (width 0.2) (layer "F.Cu") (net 11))
 (via (at 143.2 118.8) (size 0.6) (drill 0.3) (layers "F.Cu" "B.Cu") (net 11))
 (via (at 141.3 118.8) (size 0.6) (drill 0.3) (layers "F.Cu" "B.Cu") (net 11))
 (segment (start 143.2 118.8) (end 141.3 118.8) (width 0.2) (layer "B.Cu") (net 11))
 (segment (start 149.3 106.86) (end 147.91 105.47) (width 0.2) (layer "F.Cu") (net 8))
 (segment (start 145.38 120.94) (end 146.76 119.56) (width 0.2) (layer "F.Cu") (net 8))
 (segment (start 149.3 106.86) (end 148.15 108.01) (width 0.2) (layer "F.Cu") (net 8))
 (segment (start 148.15 108.01) (end 148.15 110.55) (width 0.2) (layer "F.Cu") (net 8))
 (segment (start 148.01 131.01) (end 148.01 128.47) (width 0.4) (layer "F.Cu") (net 8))
 (segment (start 148.05 125.93) (end 148.05 120.85) (width 0.4) (layer "F.Cu") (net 8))
 (segment (start 142.31 116.39) (end 142.31 119.97) (width 0.2) (layer "F.Cu") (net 8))
 (segment (start 130.355 121.315) (end 127.38 121.315) (width 2) (layer "F.Cu") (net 8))
 (segment (start 148.05 120.85) (end 146.76 119.56) (width 0.4) (layer "F.Cu") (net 8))
 (segment (start 134.77 125.73) (end 141.3 132.26) (width 2) (layer "F.Cu") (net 8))
 (segment (start 141.3 132.26) (end 146.76 132.26) (width 2) (layer "F.Cu") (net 8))
 (segment (start 142.31 119.97) (end 143.28 120.94) (width 0.2) (layer "F.Cu") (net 8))
 (segment (start 148.15 110.55) (end 146.76 111.94) (width 0.2) (layer "F.Cu") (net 8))
 (segment (start 149.3 127.18) (end 148.05 125.93) (width 0.4) (layer "F.Cu") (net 8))
 (segment (start 143.28 120.94) (end 145.38 120.94) (width 0.2) (layer "F.Cu") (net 8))
 (segment (start 141.3 133.63) (end 145.01 137.34) (width 2) (layer "F.Cu") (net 8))
 (segment (start 146.76 132.26) (end 148.01 131.01) (width 0.4) (layer "F.Cu") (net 8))
 (segment (start 148.01 128.47) (end 149.3 127.18) (width 0.4) (layer "F.Cu") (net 8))
 (segment (start 147.91 105.47) (end 147.91 102.93) (width 0.2) (layer "F.Cu") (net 8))
 (segment (start 147.91 102.93) (end 146.76 101.78) (width 0.2) (layer "F.Cu") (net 8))
 (segment (start 100.3 128.3) (end 132.2 128.3) (width 2) (layer "F.Cu") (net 8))
 (segment (start 132.2 128.3) (end 134.77 125.73) (width 2) (layer "F.Cu") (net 8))
 (segment (start 134.77 125.73) (end 130.355 121.315) (width 2) (layer "F.Cu") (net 8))
 (segment (start 145.01 137.34) (end 146.76 137.34) (width 2) (layer "F.Cu") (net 8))
 (segment (start 148.01 138.59) (end 148.01 143.67) (width 0.4) (layer "F.Cu") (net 8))
 (segment (start 146.76 137.34) (end 148.01 138.59) (width 0.4) (layer "F.Cu") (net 8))
 (segment (start 143.36 101.78) (end 139.5 97.92) (width 0.4) (layer "F.Cu") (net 8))
 (segment (start 141.3 132.26) (end 141.3 133.63) (width 2) (layer "F.Cu") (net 8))
 (segment (start 146.76 111.94) (end 142.31 116.39) (width 0.2) (layer "F.Cu") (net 8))
 (segment (start 146.76 101.78) (end 143.36 101.78) (width 0.4) (layer "F.Cu") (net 8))
 (segment (start 148.01 143.67) (end 149.3 144.96) (width 0.4) (layer "F.Cu") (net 8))
 (segment (start 145.48 125.9) (end 146.76 127.18) (width 0.2) (layer "B.Cu") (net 12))
 (segment (start 124.84 125.14) (end 125.6 125.9) (width 0.2) (layer "B.Cu") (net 12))
 (segment (start 124.84 123.855) (end 124.84 125.14) (width 0.2) (layer "B.Cu") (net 12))
 (segment (start 125.6 125.9) (end 145.48 125.9) (width 0.2) (layer "B.Cu") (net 12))
 (segment (start 124.625 126.61) (end 115.35 126.61) (width 0.7) (layer "F.Cu") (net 10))
 (segment (start 115.35 126.61) (end 113.39 124.65) (width 0.7) (layer "F.Cu") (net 10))
 (segment (start 127.38 123.855) (end 124.625 126.61) (width 0.7) (layer "F.Cu") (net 10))
 (segment (start 113.39 124.65) (end 113.39 119.38) (width 0.7) (layer "F.Cu") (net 10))
 (segment (start 133.83 98.94) (end 135.71 98.94) (width 0.7) (layer "F.Cu") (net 10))
 (segment (start 113.39 119.38) (end 133.83 98.94) (width 0.7) (layer "F.Cu") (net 10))
 (via (at 135.71 98.94) (size 0.6) (drill 0.3) (layers "F.Cu" "B.Cu") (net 10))
 (segment (start 135.71 93.04) (end 136.93 91.82) (width 0.7) (layer "B.Cu") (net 10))
 (segment (start 136.93 91.82) (end 144.42 91.82) (width 0.7) (layer "B.Cu") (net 10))
 (segment (start 144.42 91.82) (end 149.3 96.7) (width 0.7) (layer "B.Cu") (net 10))
 (segment (start 135.71 98.94) (end 135.71 93.04) (width 0.7) (layer "B.Cu") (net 10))
 (segment (start 103.4 113) (end 103.4 115.4) (width 0.2) (layer "F.Cu") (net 2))
 (segment (start 106.56 105.25) (end 100.51 111.3) (width 0.2) (layer "F.Cu") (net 2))
 (segment (start 100.3 111.3) (end 101.7 111.3) (width 0.2) (layer "F.Cu") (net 2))
 (segment (start 101.7 111.3) (end 103.4 113) (width 0.2) (layer "F.Cu") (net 2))
 (segment (start 100.51 111.3) (end 100.3 111.3) (width 0.2) (layer "F.Cu") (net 2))
 (segment (start 103.4 115.4) (end 100.3 118.5) (width 0.2) (layer "F.Cu") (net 2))
 (segment (start 98.5 114.9) (end 96.8 113.2) (width 0.2) (layer "F.Cu") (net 1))
 (segment (start 106.56 100.75) (end 100.3 107.01) (width 0.2) (layer "F.Cu") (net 1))
 (segment (start 100.3 107.01) (end 100.3 107.7) (width 0.2) (layer "F.Cu") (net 1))
 (segment (start 96.8 113.2) (end 96.8 110.2) (width 0.2) (layer "F.Cu") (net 1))
 (segment (start 100.3 114.9) (end 98.5 114.9) (width 0.2) (layer "F.Cu") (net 1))
 (segment (start 96.8 110.2) (end 99.3 107.7) (width 0.2) (layer "F.Cu") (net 1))
 (segment (start 99.3 107.7) (end 100.3 107.7) (width 0.2) (layer "F.Cu") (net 1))
 (segment (start 138.075 103) (end 119.76 121.315) (width 0.2) (layer "F.Cu") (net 6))
 (segment (start 139.5 103) (end 138.075 103) (width 0.2) (layer "F.Cu") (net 6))
 (segment (start 144 105.6) (end 144 113.1) (width 0.2) (layer "F.Cu") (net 6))
 (via (at 144 113.1) (size 0.6) (drill 0.3) (layers "F.Cu" "B.Cu") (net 6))
 (via (at 144 105.6) (size 0.6) (drill 0.3) (layers "F.Cu" "B.Cu") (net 6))
 (segment (start 146.453654 115.8) (end 149.706346 115.8) (width 0.2) (layer "B.Cu") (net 6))
 (segment (start 149.706346 115.8) (end 150.5 116.593654) (width 0.2) (layer "B.Cu") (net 6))
 (segment (start 139.5 103) (end 141.4 103) (width 0.2) (layer "B.Cu") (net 6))
 (segment (start 150.5 116.593654) (end 150.5 120.9) (width 0.2) (layer "B.Cu") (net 6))
 (segment (start 144 113.1) (end 144 113.346346) (width 0.2) (layer "B.Cu") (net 6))
 (segment (start 150.5 120.9) (end 149.3 122.1) (width 0.2) (layer "B.Cu") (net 6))
 (segment (start 141.4 103) (end 144 105.6) (width 0.2) (layer "B.Cu") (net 6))
 (segment (start 144 113.346346) (end 146.453654 115.8) (width 0.2) (layer "B.Cu") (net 6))
 (segment (start 125 117.3) (end 125 117.2) (width 0.2) (layer "B.Cu") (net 4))
 (segment (start 151.001428 108.501428) (end 151.001428 122.938572) (width 0.2) (layer "B.Cu") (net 4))
 (segment (start 129.1 118.5) (end 139.5 108.1) (width 0.2) (layer "B.Cu") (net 4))
 (segment (start 122.3 121.315) (end 122.3 120) (width 0.2) (layer "B.Cu") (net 4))
 (segment (start 151.001428 122.938572) (end 149.3 124.64) (width 0.2) (layer "B.Cu") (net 4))
 (segment (start 125.7 117.2) (end 127 118.5) (width 0.2) (layer "B.Cu") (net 4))
 (segment (start 150.58 108.08) (end 151.001428 108.501428) (width 0.2) (layer "B.Cu") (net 4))
 (segment (start 122.3 120) (end 125 117.3) (width 0.2) (layer "B.Cu") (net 4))
 (segment (start 127 118.5) (end 129.1 118.5) (width 0.2) (layer "B.Cu") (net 4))
 (segment (start 125 117.2) (end 125.7 117.2) (width 0.2) (layer "B.Cu") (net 4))
 (segment (start 139.5 108.08) (end 150.58 108.08) (width 0.2) (layer "B.Cu") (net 4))
 (segment (start 139.5 108.1) (end 139.5 108.08) (width 0.2) (layer "B.Cu") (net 4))
 (segment (start 122.3 123.855) (end 123.64 122.515) (width 0.2) (layer "F.Cu") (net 5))
 (segment (start 123.64 120.76) (end 134 110.4) (width 0.2) (layer "F.Cu") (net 5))
 (segment (start 134 110.4) (end 138.86 105.54) (width 0.2) (layer "F.Cu") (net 5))
 (segment (start 137.7 114.1) (end 134 110.4) (width 0.2) (layer "F.Cu") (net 5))
 (segment (start 139.5 114.1) (end 137.7 114.1) (width 0.2) (layer "F.Cu") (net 5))
 (segment (start 138.86 105.54) (end 139.5 105.54) (width 0.2) (layer "F.Cu") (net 5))
 (segment (start 123.64 122.515) (end 123.64 120.76) (width 0.2) (layer "F.Cu") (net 5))
 (via (at 139.5 114.1) (size 0.6) (drill 0.3) (layers "F.Cu" "B.Cu") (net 5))
 (segment (start 149.3 119.56) (end 148.04 118.3) (width 0.2) (layer "B.Cu") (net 5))
 (segment (start 148.04 118.3) (end 145.1 118.3) (width 0.2) (layer "B.Cu") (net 5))
 (segment (start 140.9 114.1) (end 139.5 114.1) (width 0.2) (layer "B.Cu") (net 5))
 (segment (start 145.1 118.3) (end 140.9 114.1) (width 0.2) (layer "B.Cu") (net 5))
 (segment (start 142.2 103.1) (end 139.56 100.46) (width 0.2) (layer "F.Cu") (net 7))
 (segment (start 140.5 116) (end 142.2 114.3) (width 0.2) (layer "F.Cu") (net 7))
 (segment (start 139.56 100.46) (end 139.5 100.46) (width 0.2) (layer "F.Cu") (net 7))
 (segment (start 140.5 117.8) (end 140.5 116) (width 0.2) (layer "F.Cu") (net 7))
 (segment (start 142.2 114.3) (end 142.2 103.1) (width 0.2) (layer "F.Cu") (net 7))
 (via (at 140.5 117.8) (size 0.6) (drill 0.3) (layers "F.Cu" "B.Cu") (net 7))
 (segment (start 141.84 124.64) (end 140.5 123.3) (width 0.2) (layer "B.Cu") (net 7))
 (segment (start 146.76 124.64) (end 141.84 124.64) (width 0.2) (layer "B.Cu") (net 7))
 (segment (start 140.5 123.3) (end 140.5 117.8) (width 0.2) (layer "B.Cu") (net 7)))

